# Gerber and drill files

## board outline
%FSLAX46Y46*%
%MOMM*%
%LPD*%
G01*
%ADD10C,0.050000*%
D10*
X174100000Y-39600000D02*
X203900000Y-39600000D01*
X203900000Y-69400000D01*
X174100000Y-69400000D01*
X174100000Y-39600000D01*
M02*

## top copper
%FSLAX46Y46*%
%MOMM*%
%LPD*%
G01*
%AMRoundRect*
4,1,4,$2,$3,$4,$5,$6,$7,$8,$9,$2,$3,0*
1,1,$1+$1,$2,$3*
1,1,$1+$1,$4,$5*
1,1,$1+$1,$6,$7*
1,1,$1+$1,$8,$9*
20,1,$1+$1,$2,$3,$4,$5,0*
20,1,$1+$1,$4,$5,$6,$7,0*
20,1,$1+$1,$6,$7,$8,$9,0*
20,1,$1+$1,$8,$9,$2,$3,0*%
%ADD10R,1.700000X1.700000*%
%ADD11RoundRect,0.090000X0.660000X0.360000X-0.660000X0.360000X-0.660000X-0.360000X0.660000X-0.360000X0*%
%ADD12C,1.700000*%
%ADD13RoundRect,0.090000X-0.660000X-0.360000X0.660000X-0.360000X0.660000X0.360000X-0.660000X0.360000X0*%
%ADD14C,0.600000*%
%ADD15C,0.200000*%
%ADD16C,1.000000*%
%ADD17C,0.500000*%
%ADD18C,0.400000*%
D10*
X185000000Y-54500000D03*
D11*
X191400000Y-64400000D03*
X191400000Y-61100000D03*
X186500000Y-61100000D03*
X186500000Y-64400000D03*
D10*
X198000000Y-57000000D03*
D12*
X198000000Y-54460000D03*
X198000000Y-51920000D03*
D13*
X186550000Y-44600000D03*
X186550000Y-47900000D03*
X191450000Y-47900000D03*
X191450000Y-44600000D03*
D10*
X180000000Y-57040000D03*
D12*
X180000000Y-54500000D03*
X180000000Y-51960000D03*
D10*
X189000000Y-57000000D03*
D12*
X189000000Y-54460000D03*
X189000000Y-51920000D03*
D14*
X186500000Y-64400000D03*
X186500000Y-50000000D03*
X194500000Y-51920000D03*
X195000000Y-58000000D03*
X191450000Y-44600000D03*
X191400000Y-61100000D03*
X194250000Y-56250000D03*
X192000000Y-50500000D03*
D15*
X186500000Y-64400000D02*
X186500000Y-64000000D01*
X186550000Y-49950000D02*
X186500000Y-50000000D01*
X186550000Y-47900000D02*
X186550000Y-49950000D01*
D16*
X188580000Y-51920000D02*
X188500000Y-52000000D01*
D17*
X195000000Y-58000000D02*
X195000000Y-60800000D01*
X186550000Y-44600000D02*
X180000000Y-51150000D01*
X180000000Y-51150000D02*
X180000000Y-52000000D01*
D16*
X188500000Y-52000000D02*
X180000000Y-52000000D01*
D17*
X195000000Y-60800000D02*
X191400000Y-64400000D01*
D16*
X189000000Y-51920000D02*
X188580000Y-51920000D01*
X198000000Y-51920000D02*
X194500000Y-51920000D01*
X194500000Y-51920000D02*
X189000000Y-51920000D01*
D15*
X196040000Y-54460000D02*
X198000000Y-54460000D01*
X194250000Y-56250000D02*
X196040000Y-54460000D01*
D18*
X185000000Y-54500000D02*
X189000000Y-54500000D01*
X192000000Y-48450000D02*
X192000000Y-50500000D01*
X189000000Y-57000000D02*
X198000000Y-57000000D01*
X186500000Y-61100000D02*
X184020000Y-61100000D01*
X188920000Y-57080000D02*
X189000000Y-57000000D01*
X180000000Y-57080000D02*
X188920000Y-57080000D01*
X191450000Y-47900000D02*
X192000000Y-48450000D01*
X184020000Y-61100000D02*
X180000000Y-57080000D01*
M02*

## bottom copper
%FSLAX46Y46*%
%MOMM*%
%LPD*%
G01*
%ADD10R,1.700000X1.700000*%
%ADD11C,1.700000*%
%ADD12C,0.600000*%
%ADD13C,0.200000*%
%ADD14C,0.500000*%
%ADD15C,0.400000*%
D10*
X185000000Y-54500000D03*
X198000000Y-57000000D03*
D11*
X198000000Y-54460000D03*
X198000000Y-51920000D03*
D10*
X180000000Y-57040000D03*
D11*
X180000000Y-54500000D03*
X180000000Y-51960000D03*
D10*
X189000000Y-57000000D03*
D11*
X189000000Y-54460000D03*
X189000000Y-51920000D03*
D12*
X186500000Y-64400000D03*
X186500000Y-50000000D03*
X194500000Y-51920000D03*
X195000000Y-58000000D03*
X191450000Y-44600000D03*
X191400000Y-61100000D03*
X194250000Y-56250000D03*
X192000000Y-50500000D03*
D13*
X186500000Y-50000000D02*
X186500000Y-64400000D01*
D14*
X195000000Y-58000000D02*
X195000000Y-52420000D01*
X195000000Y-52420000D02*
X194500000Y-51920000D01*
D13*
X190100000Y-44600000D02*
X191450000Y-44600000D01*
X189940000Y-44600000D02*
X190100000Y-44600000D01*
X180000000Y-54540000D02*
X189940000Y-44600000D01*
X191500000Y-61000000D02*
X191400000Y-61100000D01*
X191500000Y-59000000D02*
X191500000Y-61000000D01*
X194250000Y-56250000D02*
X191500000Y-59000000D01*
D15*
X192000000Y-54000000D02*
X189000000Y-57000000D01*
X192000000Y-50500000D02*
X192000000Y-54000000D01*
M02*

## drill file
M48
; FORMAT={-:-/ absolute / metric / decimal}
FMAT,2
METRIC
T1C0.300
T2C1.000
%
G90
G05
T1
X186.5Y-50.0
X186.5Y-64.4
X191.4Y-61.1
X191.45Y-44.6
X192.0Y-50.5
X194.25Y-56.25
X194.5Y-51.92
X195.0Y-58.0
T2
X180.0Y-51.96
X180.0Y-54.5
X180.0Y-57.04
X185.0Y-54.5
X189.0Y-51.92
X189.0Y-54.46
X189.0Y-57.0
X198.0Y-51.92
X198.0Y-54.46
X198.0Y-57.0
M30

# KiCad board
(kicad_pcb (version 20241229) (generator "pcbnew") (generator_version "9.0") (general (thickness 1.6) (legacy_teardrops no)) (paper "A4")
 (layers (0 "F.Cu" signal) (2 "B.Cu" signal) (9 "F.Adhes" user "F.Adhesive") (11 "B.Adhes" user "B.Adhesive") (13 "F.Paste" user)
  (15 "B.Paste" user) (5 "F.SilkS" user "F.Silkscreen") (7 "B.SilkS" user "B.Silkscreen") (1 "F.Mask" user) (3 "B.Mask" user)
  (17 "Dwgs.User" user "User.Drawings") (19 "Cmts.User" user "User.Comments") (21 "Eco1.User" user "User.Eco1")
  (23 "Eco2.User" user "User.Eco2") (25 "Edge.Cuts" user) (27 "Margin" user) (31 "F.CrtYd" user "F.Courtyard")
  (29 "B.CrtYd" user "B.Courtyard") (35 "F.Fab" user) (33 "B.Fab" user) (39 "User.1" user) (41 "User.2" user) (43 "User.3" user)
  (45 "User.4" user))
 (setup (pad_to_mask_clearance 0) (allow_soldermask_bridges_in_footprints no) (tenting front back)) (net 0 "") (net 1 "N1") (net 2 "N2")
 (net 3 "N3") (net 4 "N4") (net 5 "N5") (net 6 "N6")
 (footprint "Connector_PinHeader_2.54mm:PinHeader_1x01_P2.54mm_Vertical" (layer "F.Cu") (at 185 54.5)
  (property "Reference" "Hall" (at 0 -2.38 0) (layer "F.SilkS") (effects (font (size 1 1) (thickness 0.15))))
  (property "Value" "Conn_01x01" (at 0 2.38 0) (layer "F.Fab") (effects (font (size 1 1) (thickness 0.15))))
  (pad "1" thru_hole rect (at 0 0) (size 1.7 1.7) (drill 1) (layers "*.Cu" "*.Mask") (remove_unused_layers no) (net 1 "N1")))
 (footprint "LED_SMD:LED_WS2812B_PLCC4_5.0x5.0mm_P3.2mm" (layer "F.Cu") (at 188.95 62.75 180)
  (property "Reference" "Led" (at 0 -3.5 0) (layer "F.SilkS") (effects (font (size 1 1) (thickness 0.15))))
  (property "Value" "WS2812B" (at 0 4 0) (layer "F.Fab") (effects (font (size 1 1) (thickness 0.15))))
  (pad "1" smd roundrect (at -2.45 -1.65 180) (size 1.5 0.9) (layers "F.Cu" "F.Mask" "F.Paste") (roundrect_rratio 0.1) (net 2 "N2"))
  (pad "2" smd roundrect (at -2.45 1.65 180) (size 1.5 0.9) (layers "F.Cu" "F.Mask" "F.Paste") (roundrect_rratio 0.1) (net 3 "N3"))
  (pad "3" smd roundrect (at 2.45 1.65 180) (size 1.5 0.9) (layers "F.Cu" "F.Mask" "F.Paste") (roundrect_rratio 0.1) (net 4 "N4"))
  (pad "4" smd roundrect (at 2.45 -1.65 180) (size 1.5 0.9) (layers "F.Cu" "F.Mask" "F.Paste") (roundrect_rratio 0.1) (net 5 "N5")))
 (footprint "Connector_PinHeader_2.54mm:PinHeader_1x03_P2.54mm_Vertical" (layer "F.Cu") (at 198 57 180)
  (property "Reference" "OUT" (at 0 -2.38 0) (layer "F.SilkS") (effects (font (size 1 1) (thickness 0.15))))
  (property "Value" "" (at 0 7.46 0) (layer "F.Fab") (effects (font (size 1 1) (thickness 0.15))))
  (pad "1" thru_hole rect (at 0 0 180) (size 1.7 1.7) (drill 1) (layers "*.Cu" "*.Mask") (remove_unused_layers no) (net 4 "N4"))
  (pad "2" thru_hole circle (at 0 2.54 180) (size 1.7 1.7) (drill 1) (layers "*.Cu" "*.Mask") (remove_unused_layers no) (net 3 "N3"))
  (pad "3" thru_hole circle (at 0 5.08 180) (size 1.7 1.7) (drill 1) (layers "*.Cu" "*.Mask") (remove_unused_layers no) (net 2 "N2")))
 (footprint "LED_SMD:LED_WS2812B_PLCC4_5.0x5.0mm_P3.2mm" (layer "F.Cu") (at 189 46.25)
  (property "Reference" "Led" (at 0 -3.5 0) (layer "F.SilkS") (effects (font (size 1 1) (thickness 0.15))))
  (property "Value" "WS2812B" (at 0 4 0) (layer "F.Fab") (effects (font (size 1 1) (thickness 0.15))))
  (pad "1" smd roundrect (at -2.45 -1.65) (size 1.5 0.9) (layers "F.Cu" "F.Mask" "F.Paste") (roundrect_rratio 0.1) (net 2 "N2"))
  (pad "2" smd roundrect (at -2.45 1.65) (size 1.5 0.9) (layers "F.Cu" "F.Mask" "F.Paste") (roundrect_rratio 0.1) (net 5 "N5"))
  (pad "3" smd roundrect (at 2.45 1.65) (size 1.5 0.9) (layers "F.Cu" "F.Mask" "F.Paste") (roundrect_rratio 0.1) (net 4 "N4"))
  (pad "4" smd roundrect (at 2.45 -1.65) (size 1.5 0.9) (layers "F.Cu" "F.Mask" "F.Paste") (roundrect_rratio 0.1) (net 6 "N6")))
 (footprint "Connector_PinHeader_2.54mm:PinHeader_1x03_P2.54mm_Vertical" (layer "F.Cu") (at 180 57.04 180)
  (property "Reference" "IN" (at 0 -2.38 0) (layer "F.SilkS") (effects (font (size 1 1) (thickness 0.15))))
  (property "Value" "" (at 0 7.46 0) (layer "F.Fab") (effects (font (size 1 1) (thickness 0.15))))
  (pad "1" thru_hole rect (at 0 0 180) (size 1.7 1.7) (drill 1) (layers "*.Cu" "*.Mask") (remove_unused_layers no) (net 4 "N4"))
  (pad "2" thru_hole circle (at 0 2.54 180) (size 1.7 1.7) (drill 1) (layers "*.Cu" "*.Mask") (remove_unused_layers no) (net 6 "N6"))
  (pad "3" thru_hole circle (at 0 5.08 180) (size 1.7 1.7) (drill 1) (layers "*.Cu" "*.Mask") (remove_unused_layers no) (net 2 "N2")))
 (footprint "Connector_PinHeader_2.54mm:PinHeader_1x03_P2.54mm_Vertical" (layer "F.Cu") (at 189 57 180)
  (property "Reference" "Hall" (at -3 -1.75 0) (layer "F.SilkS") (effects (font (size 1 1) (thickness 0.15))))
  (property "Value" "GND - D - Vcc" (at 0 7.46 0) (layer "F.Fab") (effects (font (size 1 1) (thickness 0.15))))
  (pad "1" thru_hole rect (at 0 0 180) (size 1.7 1.7) (drill 1) (layers "*.Cu" "*.Mask") (remove_unused_layers no) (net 4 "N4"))
  (pad "2" thru_hole circle (at 0 2.54 180) (size 1.7 1.7) (drill 1) (layers "*.Cu" "*.Mask") (remove_unused_layers no) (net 1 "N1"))
  (pad "3" thru_hole circle (at 0 5.08 180) (size 1.7 1.7) (drill 1) (layers "*.Cu" "*.Mask") (remove_unused_layers no) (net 2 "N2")))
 (gr_rect (start 174.1 39.6) (end 203.9 69.4) (stroke (width 0.05) (type default)) (fill no) (layer "Edge.Cuts"))
 (segment (start 186.5 64.4) (end 186.5 64) (width 0.2) (layer "F.Cu") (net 5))
 (segment (start 186.55 49.95) (end 186.5 50) (width 0.2) (layer "F.Cu") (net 5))
 (segment (start 186.55 47.9) (end 186.55 49.95) (width 0.2) (layer "F.Cu") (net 5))
 (via (at 186.5 64.4) (size 0.6) (drill 0.3) (layers "F.Cu" "B.Cu") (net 5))
 (via (at 186.5 50) (size 0.6) (drill 0.3) (layers "F.Cu" "B.Cu") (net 5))
 (segment (start 186.5 50) (end 186.5 64.4) (width 0.2) (layer "B.Cu") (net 5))
 (segment (start 188.58 51.92) (end 188.5 52) (width 1) (layer "F.Cu") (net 2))
 (segment (start 195 58) (end 195 60.8) (width 0.5) (layer "F.Cu") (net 2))
 (segment (start 186.55 44.6) (end 180 51.15) (width 0.5) (layer "F.Cu") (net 2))
 (segment (start 180 51.15) (end 180 52) (width 0.5) (layer "F.Cu") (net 2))
 (segment (start 188.5 52) (end 180 52) (width 1) (layer "F.Cu") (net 2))
 (segment (start 195 60.8) (end 191.4 64.4) (width 0.5) (layer "F.Cu") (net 2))
 (segment (start 189 51.92) (end 188.58 51.92) (width 1) (layer "F.Cu") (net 2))
 (segment (start 198 51.92) (end 194.5 51.92) (width 1) (layer "F.Cu") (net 2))
 (segment (start 194.5 51.92) (end 189 51.92) (width 1) (layer "F.Cu") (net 2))
 (via (at 194.5 51.92) (size 0.6) (drill 0.3) (layers "F.Cu" "B.Cu") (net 2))
 (via (at 195 58) (size 0.6) (drill 0.3) (layers "F.Cu" "B.Cu") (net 2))
 (segment (start 195 58) (end 195 52.42) (width 0.5) (layer "B.Cu") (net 2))
 (segment (start 195 52.42) (end 194.5 51.92) (width 0.5) (layer "B.Cu") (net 2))
 (via (at 191.45 44.6) (size 0.6) (drill 0.3) (layers "F.Cu" "B.Cu") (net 6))
 (segment (start 190.1 44.6) (end 191.45 44.6) (width 0.2) (layer "B.Cu") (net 6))
 (segment (start 189.94 44.6) (end 190.1 44.6) (width 0.2) (layer "B.Cu") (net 6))
 (segment (start 180 54.54) (end 189.94 44.6) (width 0.2) (layer "B.Cu") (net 6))
 (segment (start 196.04 54.46) (end 198 54.46) (width 0.2) (layer "F.Cu") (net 3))
 (segment (start 194.25 56.25) (end 196.04 54.46) (width 0.2) (layer "F.Cu") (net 3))
 (via (at 191.4 61.1) (size 0.6) (drill 0.3) (layers "F.Cu" "B.Cu") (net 3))
 (via (at 194.25 56.25) (size 0.6) (drill 0.3) (layers "F.Cu" "B.Cu") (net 3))
 (segment (start 191.5 61) (end 191.4 61.1) (width 0.2) (layer "B.Cu") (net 3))
 (segment (start 191.5 59) (end 191.5 61) (width 0.2) (layer "B.Cu") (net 3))
 (segment (start 194.25 56.25) (end 191.5 59) (width 0.2) (layer "B.Cu") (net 3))
 (segment (start 185 54.5) (end 189 54.5) (width 0.4) (layer "F.Cu") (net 1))
 (segment (start 192 48.45) (end 192 50.5) (width 0.4) (layer "F.Cu") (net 4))
 (segment (start 189 57) (end 198 57) (width 0.4) (layer "F.Cu") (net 4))
 (segment (start 186.5 61.1) (end 184.02 61.1) (width 0.4) (layer "F.Cu") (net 4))
 (segment (start 188.92 57.08) (end 189 57) (width 0.4) (layer "F.Cu") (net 4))
 (segment (start 180 57.08) (end 188.92 57.08) (width 0.4) (layer "F.Cu") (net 4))
 (segment (start 191.45 47.9) (end 192 48.45) (width 0.4) (layer "F.Cu") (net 4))
 (segment (start 184.02 61.1) (end 180 57.08) (width 0.4) (layer "F.Cu") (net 4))
 (via (at 192 50.5) (size 0.6) (drill 0.3) (layers "F.Cu" "B.Cu") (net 4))
 (segment (start 192 54) (end 189 57) (width 0.4) (layer "B.Cu") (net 4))
 (segment (start 192 50.5) (end 192 54) (width 0.4) (layer "B.Cu") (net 4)))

